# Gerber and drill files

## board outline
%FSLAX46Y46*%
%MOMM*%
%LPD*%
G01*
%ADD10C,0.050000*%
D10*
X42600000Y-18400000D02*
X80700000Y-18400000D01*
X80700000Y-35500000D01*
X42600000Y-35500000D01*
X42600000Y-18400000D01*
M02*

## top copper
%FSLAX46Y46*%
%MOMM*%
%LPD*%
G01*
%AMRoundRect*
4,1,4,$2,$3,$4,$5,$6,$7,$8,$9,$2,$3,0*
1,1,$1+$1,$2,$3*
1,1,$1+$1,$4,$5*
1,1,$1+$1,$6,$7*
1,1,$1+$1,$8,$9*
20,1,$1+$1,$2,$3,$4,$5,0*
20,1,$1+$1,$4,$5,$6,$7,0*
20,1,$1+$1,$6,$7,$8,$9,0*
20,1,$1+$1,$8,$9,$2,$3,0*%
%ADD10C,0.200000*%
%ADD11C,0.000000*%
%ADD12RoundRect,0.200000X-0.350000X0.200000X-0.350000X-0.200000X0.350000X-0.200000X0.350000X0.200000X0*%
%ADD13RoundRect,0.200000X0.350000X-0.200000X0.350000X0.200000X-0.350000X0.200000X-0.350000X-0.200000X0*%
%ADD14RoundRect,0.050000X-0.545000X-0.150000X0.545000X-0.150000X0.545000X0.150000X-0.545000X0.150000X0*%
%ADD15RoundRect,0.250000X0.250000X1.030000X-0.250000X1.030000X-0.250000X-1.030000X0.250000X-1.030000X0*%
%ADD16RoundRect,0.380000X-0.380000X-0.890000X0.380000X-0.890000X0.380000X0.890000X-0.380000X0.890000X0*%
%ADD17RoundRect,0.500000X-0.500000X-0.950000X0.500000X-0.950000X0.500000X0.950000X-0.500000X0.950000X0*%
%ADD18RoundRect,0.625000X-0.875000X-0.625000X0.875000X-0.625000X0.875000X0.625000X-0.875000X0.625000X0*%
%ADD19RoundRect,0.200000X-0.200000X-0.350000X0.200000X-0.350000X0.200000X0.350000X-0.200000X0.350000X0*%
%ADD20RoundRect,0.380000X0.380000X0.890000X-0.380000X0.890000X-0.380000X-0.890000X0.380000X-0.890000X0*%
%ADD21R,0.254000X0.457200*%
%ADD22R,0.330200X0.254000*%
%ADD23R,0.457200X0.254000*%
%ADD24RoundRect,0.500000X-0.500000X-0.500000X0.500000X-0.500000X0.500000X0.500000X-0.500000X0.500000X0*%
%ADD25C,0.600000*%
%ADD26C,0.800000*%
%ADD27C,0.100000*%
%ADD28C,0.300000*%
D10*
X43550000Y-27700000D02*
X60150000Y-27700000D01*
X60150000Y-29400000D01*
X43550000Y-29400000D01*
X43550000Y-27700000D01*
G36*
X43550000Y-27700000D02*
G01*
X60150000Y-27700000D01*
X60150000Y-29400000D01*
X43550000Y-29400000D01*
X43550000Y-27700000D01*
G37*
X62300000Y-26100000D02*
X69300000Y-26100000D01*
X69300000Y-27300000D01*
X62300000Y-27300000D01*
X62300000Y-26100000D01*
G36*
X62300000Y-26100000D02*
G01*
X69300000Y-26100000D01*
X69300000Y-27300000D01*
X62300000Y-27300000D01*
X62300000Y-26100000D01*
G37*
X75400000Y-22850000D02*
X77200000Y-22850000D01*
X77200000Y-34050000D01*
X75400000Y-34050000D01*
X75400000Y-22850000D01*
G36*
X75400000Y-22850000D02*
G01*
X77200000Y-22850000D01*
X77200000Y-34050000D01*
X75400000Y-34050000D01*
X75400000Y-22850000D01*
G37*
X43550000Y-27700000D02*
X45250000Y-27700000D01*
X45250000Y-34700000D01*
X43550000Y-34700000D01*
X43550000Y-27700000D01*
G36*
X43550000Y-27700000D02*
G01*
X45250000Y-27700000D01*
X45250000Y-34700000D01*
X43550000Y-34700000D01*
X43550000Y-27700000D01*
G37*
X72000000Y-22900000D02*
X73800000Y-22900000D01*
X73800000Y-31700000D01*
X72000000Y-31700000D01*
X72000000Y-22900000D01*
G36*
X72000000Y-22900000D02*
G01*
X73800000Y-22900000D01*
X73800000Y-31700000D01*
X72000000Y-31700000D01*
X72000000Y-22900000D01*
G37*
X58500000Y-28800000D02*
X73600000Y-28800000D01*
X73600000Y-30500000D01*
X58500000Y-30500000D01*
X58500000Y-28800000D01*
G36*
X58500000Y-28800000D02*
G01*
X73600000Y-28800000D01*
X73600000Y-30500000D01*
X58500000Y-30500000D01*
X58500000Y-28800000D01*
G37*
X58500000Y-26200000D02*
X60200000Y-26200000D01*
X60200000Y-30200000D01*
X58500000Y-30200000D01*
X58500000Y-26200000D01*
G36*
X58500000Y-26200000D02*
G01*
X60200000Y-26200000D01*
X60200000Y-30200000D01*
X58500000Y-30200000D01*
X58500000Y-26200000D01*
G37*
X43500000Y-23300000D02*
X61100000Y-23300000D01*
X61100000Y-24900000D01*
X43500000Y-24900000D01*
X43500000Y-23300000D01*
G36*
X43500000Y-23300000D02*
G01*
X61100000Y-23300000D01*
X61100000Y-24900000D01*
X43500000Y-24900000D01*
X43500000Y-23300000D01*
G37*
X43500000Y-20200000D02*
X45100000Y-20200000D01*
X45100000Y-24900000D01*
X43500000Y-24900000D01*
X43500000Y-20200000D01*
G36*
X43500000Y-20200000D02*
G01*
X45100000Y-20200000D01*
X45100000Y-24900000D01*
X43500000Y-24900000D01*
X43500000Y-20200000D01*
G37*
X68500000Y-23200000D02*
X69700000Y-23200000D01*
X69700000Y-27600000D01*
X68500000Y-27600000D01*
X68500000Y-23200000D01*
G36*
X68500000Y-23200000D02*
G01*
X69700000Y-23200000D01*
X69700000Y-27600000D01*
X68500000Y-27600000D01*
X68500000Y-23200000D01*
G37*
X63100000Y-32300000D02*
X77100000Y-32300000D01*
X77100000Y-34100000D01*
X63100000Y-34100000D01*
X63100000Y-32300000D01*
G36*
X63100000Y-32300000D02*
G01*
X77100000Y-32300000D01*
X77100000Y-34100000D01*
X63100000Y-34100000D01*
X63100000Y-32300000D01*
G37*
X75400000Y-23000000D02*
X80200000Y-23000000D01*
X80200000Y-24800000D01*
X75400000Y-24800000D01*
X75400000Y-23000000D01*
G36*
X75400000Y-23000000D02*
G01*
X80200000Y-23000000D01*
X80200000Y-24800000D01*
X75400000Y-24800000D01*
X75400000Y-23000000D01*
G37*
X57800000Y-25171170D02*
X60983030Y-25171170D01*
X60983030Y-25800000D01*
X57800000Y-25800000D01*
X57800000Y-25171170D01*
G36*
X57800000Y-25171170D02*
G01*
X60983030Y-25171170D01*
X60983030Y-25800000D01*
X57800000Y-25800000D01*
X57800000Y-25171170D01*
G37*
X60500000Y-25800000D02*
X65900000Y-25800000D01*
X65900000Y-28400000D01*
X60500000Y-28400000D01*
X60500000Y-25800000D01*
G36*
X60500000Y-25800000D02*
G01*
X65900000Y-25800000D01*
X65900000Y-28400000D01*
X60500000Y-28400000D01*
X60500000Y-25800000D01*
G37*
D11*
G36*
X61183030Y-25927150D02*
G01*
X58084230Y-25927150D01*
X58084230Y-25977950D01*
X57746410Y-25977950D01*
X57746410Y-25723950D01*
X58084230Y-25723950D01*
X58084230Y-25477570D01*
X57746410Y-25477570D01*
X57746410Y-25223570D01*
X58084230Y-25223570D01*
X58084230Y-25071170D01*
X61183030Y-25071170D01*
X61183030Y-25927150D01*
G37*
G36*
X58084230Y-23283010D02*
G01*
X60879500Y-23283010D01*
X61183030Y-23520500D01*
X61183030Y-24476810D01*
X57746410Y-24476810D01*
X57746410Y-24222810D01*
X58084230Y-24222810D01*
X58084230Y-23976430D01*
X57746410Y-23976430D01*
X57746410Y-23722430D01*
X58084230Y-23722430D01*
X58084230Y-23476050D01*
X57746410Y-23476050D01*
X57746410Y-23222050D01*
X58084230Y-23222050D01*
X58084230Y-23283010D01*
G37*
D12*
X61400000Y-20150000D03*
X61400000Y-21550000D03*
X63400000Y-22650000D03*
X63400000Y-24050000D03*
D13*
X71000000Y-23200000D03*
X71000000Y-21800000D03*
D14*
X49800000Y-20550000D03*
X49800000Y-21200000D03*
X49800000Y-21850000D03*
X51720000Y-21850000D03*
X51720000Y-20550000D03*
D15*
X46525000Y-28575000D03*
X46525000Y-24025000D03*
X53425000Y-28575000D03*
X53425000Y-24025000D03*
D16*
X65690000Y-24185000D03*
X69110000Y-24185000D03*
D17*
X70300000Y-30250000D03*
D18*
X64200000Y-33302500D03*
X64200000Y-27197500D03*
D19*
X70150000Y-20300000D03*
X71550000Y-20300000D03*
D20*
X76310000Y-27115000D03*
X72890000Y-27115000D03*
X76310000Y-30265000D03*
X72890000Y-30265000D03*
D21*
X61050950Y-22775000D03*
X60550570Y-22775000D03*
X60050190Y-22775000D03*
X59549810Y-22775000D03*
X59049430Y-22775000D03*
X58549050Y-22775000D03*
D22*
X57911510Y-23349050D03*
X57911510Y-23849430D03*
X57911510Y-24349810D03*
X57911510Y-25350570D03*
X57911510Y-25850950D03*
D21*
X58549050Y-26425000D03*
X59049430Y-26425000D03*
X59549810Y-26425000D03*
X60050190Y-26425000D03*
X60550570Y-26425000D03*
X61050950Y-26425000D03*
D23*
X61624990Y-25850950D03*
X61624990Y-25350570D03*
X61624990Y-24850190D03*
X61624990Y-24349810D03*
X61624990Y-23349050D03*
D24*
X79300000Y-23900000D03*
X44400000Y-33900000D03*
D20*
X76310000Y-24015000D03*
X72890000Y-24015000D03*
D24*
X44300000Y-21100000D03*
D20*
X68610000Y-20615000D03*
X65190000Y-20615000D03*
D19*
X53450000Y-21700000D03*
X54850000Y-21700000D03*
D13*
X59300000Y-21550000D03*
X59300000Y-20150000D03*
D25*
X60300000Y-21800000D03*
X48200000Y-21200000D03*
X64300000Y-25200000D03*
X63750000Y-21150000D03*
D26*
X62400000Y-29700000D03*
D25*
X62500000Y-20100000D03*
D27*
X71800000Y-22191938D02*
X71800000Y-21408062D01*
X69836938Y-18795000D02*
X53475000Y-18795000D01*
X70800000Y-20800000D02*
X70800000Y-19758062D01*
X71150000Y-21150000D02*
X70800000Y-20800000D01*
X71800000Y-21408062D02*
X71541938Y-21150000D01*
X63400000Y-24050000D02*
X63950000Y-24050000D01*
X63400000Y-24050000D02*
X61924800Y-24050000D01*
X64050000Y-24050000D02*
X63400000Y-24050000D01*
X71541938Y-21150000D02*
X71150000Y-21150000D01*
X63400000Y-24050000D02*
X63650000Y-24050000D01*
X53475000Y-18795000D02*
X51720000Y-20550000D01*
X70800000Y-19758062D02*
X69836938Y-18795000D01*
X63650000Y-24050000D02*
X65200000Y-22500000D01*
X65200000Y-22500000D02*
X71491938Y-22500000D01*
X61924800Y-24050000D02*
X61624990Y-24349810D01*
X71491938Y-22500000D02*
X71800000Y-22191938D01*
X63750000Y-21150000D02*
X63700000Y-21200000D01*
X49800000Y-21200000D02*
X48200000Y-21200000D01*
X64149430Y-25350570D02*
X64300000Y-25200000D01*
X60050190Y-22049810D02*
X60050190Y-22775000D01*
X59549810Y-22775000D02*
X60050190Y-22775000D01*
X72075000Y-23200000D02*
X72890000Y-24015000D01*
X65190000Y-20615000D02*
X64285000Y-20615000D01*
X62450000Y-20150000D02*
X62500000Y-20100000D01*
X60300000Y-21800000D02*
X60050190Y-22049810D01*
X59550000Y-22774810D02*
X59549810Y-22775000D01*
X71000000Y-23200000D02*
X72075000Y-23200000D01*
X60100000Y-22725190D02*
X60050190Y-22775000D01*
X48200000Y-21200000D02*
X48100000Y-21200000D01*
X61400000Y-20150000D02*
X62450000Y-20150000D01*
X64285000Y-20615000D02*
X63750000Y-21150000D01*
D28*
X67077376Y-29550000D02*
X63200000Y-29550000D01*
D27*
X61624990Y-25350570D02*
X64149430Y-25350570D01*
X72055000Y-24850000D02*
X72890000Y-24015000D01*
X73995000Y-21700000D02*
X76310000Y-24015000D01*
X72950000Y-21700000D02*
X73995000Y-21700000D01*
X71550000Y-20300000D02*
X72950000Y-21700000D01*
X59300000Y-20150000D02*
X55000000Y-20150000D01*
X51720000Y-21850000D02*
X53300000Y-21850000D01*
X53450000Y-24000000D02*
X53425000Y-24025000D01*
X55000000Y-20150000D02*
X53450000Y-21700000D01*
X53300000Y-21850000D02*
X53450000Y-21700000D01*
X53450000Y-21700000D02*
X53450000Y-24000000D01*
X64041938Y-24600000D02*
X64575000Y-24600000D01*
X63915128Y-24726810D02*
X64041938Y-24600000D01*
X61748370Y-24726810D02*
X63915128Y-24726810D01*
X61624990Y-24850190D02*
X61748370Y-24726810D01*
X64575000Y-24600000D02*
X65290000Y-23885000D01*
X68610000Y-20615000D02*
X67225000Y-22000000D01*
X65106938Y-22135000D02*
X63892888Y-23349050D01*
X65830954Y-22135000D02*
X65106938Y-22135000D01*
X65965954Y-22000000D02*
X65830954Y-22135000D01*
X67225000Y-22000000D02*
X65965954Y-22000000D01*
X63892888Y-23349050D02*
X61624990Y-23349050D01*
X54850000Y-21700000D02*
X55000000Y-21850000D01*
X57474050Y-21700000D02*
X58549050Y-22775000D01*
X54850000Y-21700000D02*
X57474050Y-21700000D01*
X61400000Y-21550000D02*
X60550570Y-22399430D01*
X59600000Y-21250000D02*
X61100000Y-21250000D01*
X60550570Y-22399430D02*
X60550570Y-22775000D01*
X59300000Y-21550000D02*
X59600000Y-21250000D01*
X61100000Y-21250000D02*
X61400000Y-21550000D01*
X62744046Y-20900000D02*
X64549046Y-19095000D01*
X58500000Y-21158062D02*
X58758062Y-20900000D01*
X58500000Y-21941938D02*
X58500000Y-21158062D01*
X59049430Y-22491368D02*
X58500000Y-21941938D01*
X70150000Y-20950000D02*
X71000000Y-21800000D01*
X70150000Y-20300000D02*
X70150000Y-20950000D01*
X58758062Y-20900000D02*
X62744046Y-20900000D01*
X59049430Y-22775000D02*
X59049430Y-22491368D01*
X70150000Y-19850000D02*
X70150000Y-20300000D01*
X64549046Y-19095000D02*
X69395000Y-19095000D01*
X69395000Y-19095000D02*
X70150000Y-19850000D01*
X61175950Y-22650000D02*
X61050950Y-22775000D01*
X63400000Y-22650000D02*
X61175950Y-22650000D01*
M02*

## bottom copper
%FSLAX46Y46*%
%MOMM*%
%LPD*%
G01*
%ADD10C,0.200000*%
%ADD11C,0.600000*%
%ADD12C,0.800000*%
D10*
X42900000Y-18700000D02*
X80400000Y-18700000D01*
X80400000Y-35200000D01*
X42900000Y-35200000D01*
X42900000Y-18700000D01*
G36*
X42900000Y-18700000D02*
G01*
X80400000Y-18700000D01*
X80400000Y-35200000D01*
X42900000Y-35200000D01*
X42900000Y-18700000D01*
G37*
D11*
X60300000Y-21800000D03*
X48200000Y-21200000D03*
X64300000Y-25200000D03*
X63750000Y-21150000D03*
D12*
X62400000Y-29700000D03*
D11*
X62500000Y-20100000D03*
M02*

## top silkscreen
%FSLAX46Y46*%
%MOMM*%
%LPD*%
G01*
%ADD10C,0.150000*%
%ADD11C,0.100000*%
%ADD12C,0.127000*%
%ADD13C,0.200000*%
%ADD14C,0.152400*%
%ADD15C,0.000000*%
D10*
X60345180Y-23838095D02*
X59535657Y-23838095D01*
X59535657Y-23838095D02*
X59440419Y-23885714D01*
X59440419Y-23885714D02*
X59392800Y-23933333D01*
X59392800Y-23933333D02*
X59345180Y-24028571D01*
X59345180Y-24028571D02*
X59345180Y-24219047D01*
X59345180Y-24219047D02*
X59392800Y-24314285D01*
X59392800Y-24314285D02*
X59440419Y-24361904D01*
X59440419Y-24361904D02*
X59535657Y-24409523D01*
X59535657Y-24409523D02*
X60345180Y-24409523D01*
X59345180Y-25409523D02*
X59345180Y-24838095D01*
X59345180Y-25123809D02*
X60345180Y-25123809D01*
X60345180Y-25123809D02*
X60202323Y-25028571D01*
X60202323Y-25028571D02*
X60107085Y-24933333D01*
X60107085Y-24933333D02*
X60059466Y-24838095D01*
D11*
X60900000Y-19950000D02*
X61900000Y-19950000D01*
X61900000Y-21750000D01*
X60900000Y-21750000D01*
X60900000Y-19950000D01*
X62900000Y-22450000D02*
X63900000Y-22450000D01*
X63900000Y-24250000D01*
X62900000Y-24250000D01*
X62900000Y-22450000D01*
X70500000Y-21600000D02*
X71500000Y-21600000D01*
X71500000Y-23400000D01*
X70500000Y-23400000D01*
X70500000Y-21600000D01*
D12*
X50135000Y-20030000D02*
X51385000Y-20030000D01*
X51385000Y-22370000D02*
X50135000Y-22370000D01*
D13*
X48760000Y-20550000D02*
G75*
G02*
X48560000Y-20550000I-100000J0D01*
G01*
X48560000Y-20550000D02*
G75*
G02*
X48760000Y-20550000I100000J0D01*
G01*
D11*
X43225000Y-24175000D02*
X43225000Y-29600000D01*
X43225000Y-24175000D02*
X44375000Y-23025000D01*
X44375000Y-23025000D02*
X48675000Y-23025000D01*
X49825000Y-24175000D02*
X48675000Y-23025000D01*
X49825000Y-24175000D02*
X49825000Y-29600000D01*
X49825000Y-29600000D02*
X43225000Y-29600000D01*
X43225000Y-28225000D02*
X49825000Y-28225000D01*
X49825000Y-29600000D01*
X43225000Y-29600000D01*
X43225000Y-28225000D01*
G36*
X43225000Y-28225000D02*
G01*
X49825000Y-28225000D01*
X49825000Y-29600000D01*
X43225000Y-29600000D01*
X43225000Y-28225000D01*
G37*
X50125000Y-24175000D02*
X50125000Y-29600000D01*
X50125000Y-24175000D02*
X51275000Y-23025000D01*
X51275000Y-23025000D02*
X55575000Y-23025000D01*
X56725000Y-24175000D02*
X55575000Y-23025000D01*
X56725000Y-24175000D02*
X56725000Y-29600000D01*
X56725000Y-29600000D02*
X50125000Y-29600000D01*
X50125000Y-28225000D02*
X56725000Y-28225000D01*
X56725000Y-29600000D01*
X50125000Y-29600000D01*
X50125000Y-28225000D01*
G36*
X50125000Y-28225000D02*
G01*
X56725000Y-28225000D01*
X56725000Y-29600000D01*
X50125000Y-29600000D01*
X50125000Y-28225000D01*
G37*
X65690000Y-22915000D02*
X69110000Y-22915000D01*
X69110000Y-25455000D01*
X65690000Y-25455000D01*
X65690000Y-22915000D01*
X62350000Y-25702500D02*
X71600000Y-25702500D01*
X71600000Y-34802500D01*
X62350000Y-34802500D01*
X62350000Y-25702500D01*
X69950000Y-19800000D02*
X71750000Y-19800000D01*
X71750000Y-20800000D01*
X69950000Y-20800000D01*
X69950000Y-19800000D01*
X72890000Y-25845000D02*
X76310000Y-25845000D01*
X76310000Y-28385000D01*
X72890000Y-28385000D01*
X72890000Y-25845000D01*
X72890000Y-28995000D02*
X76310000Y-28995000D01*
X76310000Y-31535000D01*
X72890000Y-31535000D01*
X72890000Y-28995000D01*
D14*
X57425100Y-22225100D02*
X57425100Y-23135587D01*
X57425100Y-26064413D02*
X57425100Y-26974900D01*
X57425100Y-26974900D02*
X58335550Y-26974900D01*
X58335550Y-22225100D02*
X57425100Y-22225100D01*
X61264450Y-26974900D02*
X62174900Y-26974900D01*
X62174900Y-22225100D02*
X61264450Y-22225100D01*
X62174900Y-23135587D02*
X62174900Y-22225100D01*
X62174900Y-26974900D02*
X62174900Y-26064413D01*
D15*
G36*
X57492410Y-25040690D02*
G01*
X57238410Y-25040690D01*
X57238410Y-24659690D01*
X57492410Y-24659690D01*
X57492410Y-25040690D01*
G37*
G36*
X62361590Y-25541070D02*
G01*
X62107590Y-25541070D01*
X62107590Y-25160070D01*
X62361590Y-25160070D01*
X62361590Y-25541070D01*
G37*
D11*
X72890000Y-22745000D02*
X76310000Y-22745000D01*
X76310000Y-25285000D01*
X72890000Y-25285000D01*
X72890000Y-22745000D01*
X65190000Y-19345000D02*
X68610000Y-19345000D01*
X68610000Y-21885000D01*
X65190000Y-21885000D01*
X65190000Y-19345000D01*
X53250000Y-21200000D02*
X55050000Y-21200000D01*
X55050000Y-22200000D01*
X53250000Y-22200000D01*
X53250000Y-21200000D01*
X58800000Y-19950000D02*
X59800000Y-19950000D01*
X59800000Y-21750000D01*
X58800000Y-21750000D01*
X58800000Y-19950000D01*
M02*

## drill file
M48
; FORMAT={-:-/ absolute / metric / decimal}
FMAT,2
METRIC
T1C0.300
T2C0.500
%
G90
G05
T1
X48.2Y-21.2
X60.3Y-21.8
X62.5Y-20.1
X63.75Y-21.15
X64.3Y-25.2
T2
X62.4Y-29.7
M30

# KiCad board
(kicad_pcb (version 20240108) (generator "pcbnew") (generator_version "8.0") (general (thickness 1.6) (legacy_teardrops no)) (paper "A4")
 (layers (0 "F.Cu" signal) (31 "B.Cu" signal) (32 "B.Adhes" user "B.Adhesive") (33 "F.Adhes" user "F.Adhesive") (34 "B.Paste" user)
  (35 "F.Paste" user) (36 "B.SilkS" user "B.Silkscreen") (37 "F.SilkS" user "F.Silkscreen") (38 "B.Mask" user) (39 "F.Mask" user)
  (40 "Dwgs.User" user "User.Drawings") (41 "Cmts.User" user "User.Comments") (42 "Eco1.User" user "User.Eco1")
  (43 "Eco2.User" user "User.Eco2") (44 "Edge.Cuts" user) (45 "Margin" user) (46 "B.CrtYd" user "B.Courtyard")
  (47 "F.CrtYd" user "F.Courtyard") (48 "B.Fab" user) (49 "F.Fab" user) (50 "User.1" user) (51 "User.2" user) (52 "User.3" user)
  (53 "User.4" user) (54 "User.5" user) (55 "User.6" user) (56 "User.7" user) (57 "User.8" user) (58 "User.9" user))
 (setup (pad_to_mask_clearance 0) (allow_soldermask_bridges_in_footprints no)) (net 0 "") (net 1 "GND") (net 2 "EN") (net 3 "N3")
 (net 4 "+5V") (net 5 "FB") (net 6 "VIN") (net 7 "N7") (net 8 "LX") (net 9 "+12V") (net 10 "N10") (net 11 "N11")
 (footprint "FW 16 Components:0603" (layer "F.Cu") (at 61.4 20.8 -90)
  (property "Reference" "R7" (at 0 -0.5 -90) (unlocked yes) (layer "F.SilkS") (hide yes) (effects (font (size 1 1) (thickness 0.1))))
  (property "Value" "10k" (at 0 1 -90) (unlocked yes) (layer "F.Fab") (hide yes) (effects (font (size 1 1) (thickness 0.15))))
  (fp_rect (start -0.85 -0.5) (end 0.95 0.5) (stroke (width 0.1) (type default)) (fill none) (layer "F.SilkS"))
  (pad "1" smd roundrect (at -0.65 0 270) (size 0.8 1.1) (layers "F.Cu" "F.Paste" "F.Mask") (roundrect_rratio 0.25) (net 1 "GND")
   (thermal_bridge_angle 45))
  (pad "2" smd roundrect (at 0.75 0 270) (size 0.8 1.1) (layers "F.Cu" "F.Paste" "F.Mask") (roundrect_rratio 0.25) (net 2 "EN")
   (thermal_bridge_angle 45)))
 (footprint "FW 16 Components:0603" (layer "F.Cu") (at 63.4 23.3 -90)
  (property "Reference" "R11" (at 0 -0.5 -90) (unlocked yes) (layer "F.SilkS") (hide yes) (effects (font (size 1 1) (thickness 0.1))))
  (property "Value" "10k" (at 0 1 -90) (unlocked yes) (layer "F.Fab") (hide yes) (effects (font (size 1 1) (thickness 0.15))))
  (fp_rect (start -0.85 -0.5) (end 0.95 0.5) (stroke (width 0.1) (type default)) (fill none) (layer "F.SilkS"))
  (pad "1" smd roundrect (at -0.65 0 270) (size 0.8 1.1) (layers "F.Cu" "F.Paste" "F.Mask") (roundrect_rratio 0.25) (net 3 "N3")
   (thermal_bridge_angle 45))
  (pad "2" smd roundrect (at 0.75 0 270) (size 0.8 1.1) (layers "F.Cu" "F.Paste" "F.Mask") (roundrect_rratio 0.25) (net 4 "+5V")
   (thermal_bridge_angle 45)))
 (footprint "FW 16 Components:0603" (layer "F.Cu") (at 71 22.55 90)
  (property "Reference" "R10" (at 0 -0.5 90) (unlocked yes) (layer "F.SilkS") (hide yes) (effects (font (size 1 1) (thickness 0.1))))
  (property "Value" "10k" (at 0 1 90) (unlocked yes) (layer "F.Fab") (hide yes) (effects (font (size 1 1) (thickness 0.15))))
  (fp_rect (start -0.85 -0.5) (end 0.95 0.5) (stroke (width 0.1) (type default)) (fill none) (layer "F.SilkS"))
  (pad "1" smd roundrect (at -0.65 0 90) (size 0.8 1.1) (layers "F.Cu" "F.Paste" "F.Mask") (roundrect_rratio 0.25) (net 1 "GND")
   (thermal_bridge_angle 45))
  (pad "2" smd roundrect (at 0.75 0 90) (size 0.8 1.1) (layers "F.Cu" "F.Paste" "F.Mask") (roundrect_rratio 0.25) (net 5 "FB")
   (thermal_bridge_angle 45)))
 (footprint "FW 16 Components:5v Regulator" (layer "F.Cu") (at 50.76 21.2)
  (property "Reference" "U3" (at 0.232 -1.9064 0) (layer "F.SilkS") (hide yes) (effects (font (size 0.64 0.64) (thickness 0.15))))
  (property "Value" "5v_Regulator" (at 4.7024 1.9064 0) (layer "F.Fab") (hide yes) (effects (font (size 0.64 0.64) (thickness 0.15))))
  (fp_line (start -0.625 -1.17) (end 0.625 -1.17) (stroke (width 0.127) (type solid)) (layer "F.SilkS"))
  (fp_line (start 0.625 1.17) (end -0.625 1.17) (stroke (width 0.127) (type solid)) (layer "F.SilkS"))
  (fp_circle (center -2.1 -0.65) (end -2 -0.65) (stroke (width 0.2) (type solid)) (fill none) (layer "F.SilkS"))
  (pad "1" smd roundrect (at -0.96 -0.65) (size 1.19 0.4) (layers "F.Cu" "F.Paste" "F.Mask") (roundrect_rratio 0.125)
   (solder_mask_margin 0.102))
  (pad "2" smd roundrect (at -0.96 0) (size 1.19 0.4) (layers "F.Cu" "F.Paste" "F.Mask") (roundrect_rratio 0.125) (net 1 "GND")
   (solder_mask_margin 0.102))
  (pad "3" smd roundrect (at -0.96 0.65) (size 1.19 0.4) (layers "F.Cu" "F.Paste" "F.Mask") (roundrect_rratio 0.125)
   (solder_mask_margin 0.102))
  (pad "4" smd roundrect (at 0.96 0.65) (size 1.19 0.4) (layers "F.Cu" "F.Paste" "F.Mask") (roundrect_rratio 0.125) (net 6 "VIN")
   (solder_mask_margin 0.102))
  (pad "5" smd roundrect (at 0.96 -0.65) (size 1.19 0.4) (layers "F.Cu" "F.Paste" "F.Mask") (roundrect_rratio 0.125) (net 4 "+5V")
   (solder_mask_margin 0.102)))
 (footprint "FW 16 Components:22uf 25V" (layer "F.Cu") (at 49.975 26.125 90)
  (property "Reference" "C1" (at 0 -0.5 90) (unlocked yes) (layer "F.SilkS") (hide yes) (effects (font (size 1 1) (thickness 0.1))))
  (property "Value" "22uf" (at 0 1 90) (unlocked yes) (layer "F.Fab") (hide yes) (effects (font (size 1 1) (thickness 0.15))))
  (fp_line (start 1.95 -6.75) (end -3.475 -6.75) (stroke (width 0.1) (type default)) (layer "F.SilkS"))
  (fp_line (start 1.95 -6.75) (end 3.1 -5.6) (stroke (width 0.1) (type default)) (layer "F.SilkS"))
  (fp_line (start 3.1 -5.6) (end 3.1 -1.3) (stroke (width 0.1) (type default)) (layer "F.SilkS"))
  (fp_line (start 1.95 -0.15) (end 3.1 -1.3) (stroke (width 0.1) (type default)) (layer "F.SilkS"))
  (fp_line (start 1.95 -0.15) (end -3.475 -0.15) (stroke (width 0.1) (type default)) (layer "F.SilkS"))
  (fp_line (start -3.475 -0.15) (end -3.475 -6.75) (stroke (width 0.1) (type default)) (layer "F.SilkS"))
  (fp_rect (start -3.475 -6.75) (end -2.1 -0.15) (stroke (width 0.1) (type solid)) (fill solid) (layer "F.SilkS"))
  (pad "1" smd roundrect (at -2.45 -3.45 180) (size 1 2.56) (layers "F.Cu" "F.Paste" "F.Mask") (roundrect_rratio 0.25) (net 1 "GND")
   (thermal_bridge_angle 45))
  (pad "2" smd roundrect (at 2.1 -3.45 180) (size 1 2.56) (layers "F.Cu" "F.Paste" "F.Mask") (roundrect_rratio 0.25) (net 6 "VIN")
   (thermal_bridge_angle 45)))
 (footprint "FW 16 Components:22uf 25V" (layer "F.Cu") (at 56.875 26.125 90)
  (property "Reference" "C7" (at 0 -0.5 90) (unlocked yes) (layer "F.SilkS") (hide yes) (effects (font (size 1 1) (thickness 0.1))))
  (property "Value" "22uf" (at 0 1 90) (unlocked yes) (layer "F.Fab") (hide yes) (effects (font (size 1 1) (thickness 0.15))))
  (fp_line (start 1.95 -6.75) (end -3.475 -6.75) (stroke (width 0.1) (type default)) (layer "F.SilkS"))
  (fp_line (start 1.95 -6.75) (end 3.1 -5.6) (stroke (width 0.1) (type default)) (layer "F.SilkS"))
  (fp_line (start 3.1 -5.6) (end 3.1 -1.3) (stroke (width 0.1) (type default)) (layer "F.SilkS"))
  (fp_line (start 1.95 -0.15) (end 3.1 -1.3) (stroke (width 0.1) (type default)) (layer "F.SilkS"))
  (fp_line (start 1.95 -0.15) (end -3.475 -0.15) (stroke (width 0.1) (type default)) (layer "F.SilkS"))
  (fp_line (start -3.475 -0.15) (end -3.475 -6.75) (stroke (width 0.1) (type default)) (layer "F.SilkS"))
  (fp_rect (start -3.475 -6.75) (end -2.1 -0.15) (stroke (width 0.1) (type solid)) (fill solid) (layer "F.SilkS"))
  (pad "1" smd roundrect (at -2.45 -3.45 180) (size 1 2.56) (layers "F.Cu" "F.Paste" "F.Mask") (roundrect_rratio 0.25) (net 1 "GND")
   (thermal_bridge_angle 45))
  (pad "2" smd roundrect (at 2.1 -3.45 180) (size 1 2.56) (layers "F.Cu" "F.Paste" "F.Mask") (roundrect_rratio 0.25) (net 6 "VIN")
   (thermal_bridge_angle 45)))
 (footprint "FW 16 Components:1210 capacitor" (layer "F.Cu") (at 67.56 26.685)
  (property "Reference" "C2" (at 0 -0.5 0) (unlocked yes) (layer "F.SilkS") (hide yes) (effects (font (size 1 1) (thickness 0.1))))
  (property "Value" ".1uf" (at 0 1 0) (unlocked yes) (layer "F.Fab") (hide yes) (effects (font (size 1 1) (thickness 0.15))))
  (fp_rect (start -1.87 -3.77) (end 1.55 -1.23) (stroke (width 0.1) (type default)) (fill none) (layer "F.SilkS"))
  (pad "1" smd roundrect (at -1.87 -2.5) (size 1.52 2.54) (layers "F.Cu" "F.Paste" "F.Mask") (roundrect_rratio 0.25) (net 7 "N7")
   (thermal_bridge_angle 45))
  (pad "2" smd roundrect (at 1.55 -2.5) (size 1.52 2.54) (layers "F.Cu" "F.Paste" "F.Mask") (roundrect_rratio 0.25) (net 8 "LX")
   (thermal_bridge_angle 45)))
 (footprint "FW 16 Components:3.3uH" (layer "F.Cu") (at 66.8 30.2)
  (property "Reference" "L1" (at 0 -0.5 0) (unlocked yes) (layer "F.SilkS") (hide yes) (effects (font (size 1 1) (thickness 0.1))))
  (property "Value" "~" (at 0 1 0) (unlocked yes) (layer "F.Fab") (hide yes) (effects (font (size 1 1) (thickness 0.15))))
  (fp_rect (start -4.45 -4.4975) (end 4.8 4.6025) (stroke (width 0.1) (type default)) (fill none) (layer "F.SilkS"))
  (pad "" smd roundrect (at 3.5 0.05) (size 2 2.9) (layers "F.Cu" "F.Paste" "F.Mask") (roundrect_rratio 0.25) (thermal_bridge_angle 45))
  (pad "1" smd roundrect (at -2.6 3.1025) (size 3 2.5) (layers "F.Cu" "F.Paste" "F.Mask") (roundrect_rratio 0.25) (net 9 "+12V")
   (thermal_bridge_angle 45))
  (pad "2" smd roundrect (at -2.6 -3.0025) (size 3 2.5) (layers "F.Cu" "F.Paste" "F.Mask") (roundrect_rratio 0.25) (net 8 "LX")
   (thermal_bridge_angle 45)))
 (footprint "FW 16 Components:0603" (layer "F.Cu") (at 70.8 20.3)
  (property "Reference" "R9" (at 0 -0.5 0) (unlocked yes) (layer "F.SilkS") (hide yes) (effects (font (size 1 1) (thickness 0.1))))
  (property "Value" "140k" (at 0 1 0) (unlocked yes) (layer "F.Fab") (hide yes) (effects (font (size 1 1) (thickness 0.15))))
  (fp_rect (start -0.85 -0.5) (end 0.95 0.5) (stroke (width 0.1) (type default)) (fill none) (layer "F.SilkS"))
  (pad "1" smd roundrect (at -0.65 0) (size 0.8 1.1) (layers "F.Cu" "F.Paste" "F.Mask") (roundrect_rratio 0.25) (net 5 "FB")
   (thermal_bridge_angle 45))
  (pad "2" smd roundrect (at 0.75 0) (size 0.8 1.1) (layers "F.Cu" "F.Paste" "F.Mask") (roundrect_rratio 0.25) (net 9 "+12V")
   (thermal_bridge_angle 45)))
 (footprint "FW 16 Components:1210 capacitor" (layer "F.Cu") (at 74.44 24.615 180)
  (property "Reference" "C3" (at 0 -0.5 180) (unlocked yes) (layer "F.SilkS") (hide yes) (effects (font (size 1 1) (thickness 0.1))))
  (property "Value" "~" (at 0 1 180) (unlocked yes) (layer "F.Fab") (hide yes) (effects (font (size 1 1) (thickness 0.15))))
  (fp_rect (start -1.87 -3.77) (end 1.55 -1.23) (stroke (width 0.1) (type default)) (fill none) (layer "F.SilkS"))
  (pad "1" smd roundrect (at -1.87 -2.5 180) (size 1.52 2.54) (layers "F.Cu" "F.Paste" "F.Mask") (roundrect_rratio 0.25) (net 9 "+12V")
   (thermal_bridge_angle 45))
  (pad "2" smd roundrect (at 1.55 -2.5 180) (size 1.52 2.54) (layers "F.Cu" "F.Paste" "F.Mask") (roundrect_rratio 0.25) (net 1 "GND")
   (thermal_bridge_angle 45)))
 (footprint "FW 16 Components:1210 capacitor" (layer "F.Cu") (at 74.44 27.765 180)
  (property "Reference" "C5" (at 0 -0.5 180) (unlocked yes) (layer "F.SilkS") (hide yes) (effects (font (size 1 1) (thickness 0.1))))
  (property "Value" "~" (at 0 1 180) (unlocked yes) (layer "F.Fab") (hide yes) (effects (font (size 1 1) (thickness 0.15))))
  (fp_rect (start -1.87 -3.77) (end 1.55 -1.23) (stroke (width 0.1) (type default)) (fill none) (layer "F.SilkS"))
  (pad "1" smd roundrect (at -1.87 -2.5 180) (size 1.52 2.54) (layers "F.Cu" "F.Paste" "F.Mask") (roundrect_rratio 0.25) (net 9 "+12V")
   (thermal_bridge_angle 45))
  (pad "2" smd roundrect (at 1.55 -2.5 180) (size 1.52 2.54) (layers "F.Cu" "F.Paste" "F.Mask") (roundrect_rratio 0.25) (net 1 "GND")
   (thermal_bridge_angle 45)))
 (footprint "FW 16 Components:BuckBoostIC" (layer "F.Cu") (at 59.8 24.6 -90)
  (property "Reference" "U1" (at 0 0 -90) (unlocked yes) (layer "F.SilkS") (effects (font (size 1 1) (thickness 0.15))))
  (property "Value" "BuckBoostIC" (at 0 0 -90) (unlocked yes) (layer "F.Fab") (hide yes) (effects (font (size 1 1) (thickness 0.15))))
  (fp_poly
   (pts (xy 0.47117 1.71577) (xy 0.62357 1.71577) (xy 0.62357 2.05359) (xy 0.87757 2.05359) (xy 0.87757 1.71577) (xy 1.12395 1.71577)
    (xy 1.12395 2.05359) (xy 1.37795 2.05359) (xy 1.37795 1.71577) (xy 1.32715 1.71577) (xy 1.32715 -1.38303) (xy 0.47117 -1.38303))
   (stroke (width 0) (type solid)) (fill solid) (layer "F.Cu"))
  (fp_poly
   (pts (xy -1.37795 2.05359) (xy -1.37795 1.71577) (xy -1.31699 1.71577) (xy -1.31699 -1.0795) (xy -1.0795 -1.38303) (xy -0.12319 -1.38303)
    (xy -0.12319 2.05359) (xy -0.37719 2.05359) (xy -0.37719 1.71577) (xy -0.62357 1.71577) (xy -0.62357 2.05359) (xy -0.87757 2.05359)
    (xy -0.87757 1.71577) (xy -1.12395 1.71577) (xy -1.12395 2.05359))
   (stroke (width 0) (type solid)) (fill solid) (layer "F.Cu"))
  (fp_line (start -2.3749 2.3749) (end -1.464413 2.3749) (stroke (width 0.1524) (type solid)) (layer "F.SilkS"))
  (fp_line (start 1.464413 2.3749) (end 2.3749 2.3749) (stroke (width 0.1524) (type solid)) (layer "F.SilkS"))
  (fp_line (start 2.3749 2.3749) (end 2.3749 1.46445) (stroke (width 0.1524) (type solid)) (layer "F.SilkS"))
  (fp_line (start -2.3749 1.46445) (end -2.3749 2.3749) (stroke (width 0.1524) (type solid)) (layer "F.SilkS"))
  (fp_line (start 2.3749 -1.46445) (end 2.3749 -2.3749) (stroke (width 0.1524) (type solid)) (layer "F.SilkS"))
  (fp_line (start -2.3749 -2.3749) (end -2.3749 -1.46445) (stroke (width 0.1524) (type solid)) (layer "F.SilkS"))
  (fp_line (start -1.464413 -2.3749) (end -2.3749 -2.3749) (stroke (width 0.1524) (type solid)) (layer "F.SilkS"))
  (fp_line (start 2.3749 -2.3749) (end 1.464413 -2.3749) (stroke (width 0.1524) (type solid)) (layer "F.SilkS"))
  (fp_poly
   (pts (xy 0.05969 2.30759) (xy 0.05969 2.56159) (xy 0.44069 2.56159) (xy 0.44069 2.30759)) (stroke (width 0) (type solid)) (fill solid)
   (layer "F.SilkS"))
  (fp_poly
   (pts (xy 0.56007 -2.30759) (xy 0.56007 -2.56159) (xy 0.94107 -2.56159) (xy 0.94107 -2.30759)) (stroke (width 0) (type solid))
   (fill solid) (layer "F.SilkS"))
  (pad "1" smd rect (at -1.825 -1.25095) (size 0.254 0.4572) (layers "F.Cu" "F.Paste" "F.Mask") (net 3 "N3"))
  (pad "2" smd rect (at -1.825 -0.75057) (size 0.254 0.4572) (layers "F.Cu" "F.Paste" "F.Mask") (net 2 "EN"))
  (pad "3" smd rect (at -1.825 -0.25019) (size 0.254 0.4572) (layers "F.Cu" "F.Paste" "F.Mask") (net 1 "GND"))
  (pad "4" smd rect (at -1.825 0.25019) (size 0.254 0.4572) (layers "F.Cu" "F.Paste" "F.Mask") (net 1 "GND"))
  (pad "5" smd rect (at -1.825 0.75057) (size 0.254 0.4572) (layers "F.Cu" "F.Paste" "F.Mask") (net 5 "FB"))
  (pad "6" smd rect (at -1.825 1.25095) (size 0.254 0.4572) (layers "F.Cu" "F.Paste" "F.Mask") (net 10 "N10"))
  (pad "7" smd rect (at -1.25095 1.88849 270) (size 0.254 0.3302) (layers "F.Cu" "F.Paste" "F.Mask") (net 6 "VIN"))
  (pad "8" smd rect (at -0.75057 1.88849 270) (size 0.254 0.3302) (layers "F.Cu" "F.Paste" "F.Mask") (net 6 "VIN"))
  (pad "9" smd rect (at -0.25019 1.88849 270) (size 0.254 0.3302) (layers "F.Cu" "F.Paste" "F.Mask") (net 6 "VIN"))
  (pad "10" smd rect (at 0.75057 1.88849 270) (size 0.254 0.3302) (layers "F.Cu" "F.Paste" "F.Mask") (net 8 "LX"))
  (pad "11" smd rect (at 1.25095 1.88849 270) (size 0.254 0.3302) (layers "F.Cu" "F.Paste" "F.Mask") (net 8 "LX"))
  (pad "12" smd rect (at 1.825 1.25095) (size 0.254 0.4572) (layers "F.Cu" "F.Paste" "F.Mask") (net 1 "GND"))
  (pad "13" smd rect (at 1.825 0.75057) (size 0.254 0.4572) (layers "F.Cu" "F.Paste" "F.Mask") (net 1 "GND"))
  (pad "14" smd rect (at 1.825 0.25019) (size 0.254 0.4572) (layers "F.Cu" "F.Paste" "F.Mask") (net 1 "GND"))
  (pad "15" smd rect (at 1.825 -0.25019) (size 0.254 0.4572) (layers "F.Cu" "F.Paste" "F.Mask") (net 1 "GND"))
  (pad "16" smd rect (at 1.825 -0.75057) (size 0.254 0.4572) (layers "F.Cu" "F.Paste" "F.Mask") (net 8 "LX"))
  (pad "17" smd rect (at 1.825 -1.25095) (size 0.254 0.4572) (layers "F.Cu" "F.Paste" "F.Mask") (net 8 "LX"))
  (pad "18" smd rect (at 1.25095 -1.82499 270) (size 0.254 0.4572) (layers "F.Cu" "F.Paste" "F.Mask") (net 8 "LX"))
  (pad "19" smd rect (at 0.75057 -1.82499 270) (size 0.254 0.4572) (layers "F.Cu" "F.Paste" "F.Mask") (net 1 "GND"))
  (pad "20" smd rect (at 0.25019 -1.82499 270) (size 0.254 0.4572) (layers "F.Cu" "F.Paste" "F.Mask") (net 7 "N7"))
  (pad "21" smd rect (at -0.25019 -1.82499 270) (size 0.254 0.4572) (layers "F.Cu" "F.Paste" "F.Mask") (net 4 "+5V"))
  (pad "22" smd rect (at -1.25095 -1.82499 270) (size 0.254 0.4572) (layers "F.Cu" "F.Paste" "F.Mask") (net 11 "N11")))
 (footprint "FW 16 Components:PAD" (layer "F.Cu") (at 79.35 26.45)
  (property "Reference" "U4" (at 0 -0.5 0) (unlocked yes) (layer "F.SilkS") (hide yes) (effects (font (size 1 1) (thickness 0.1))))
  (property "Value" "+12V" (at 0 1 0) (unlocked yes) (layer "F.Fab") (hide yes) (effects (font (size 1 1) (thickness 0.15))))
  (pad "1" smd roundrect (at -0.05 -2.55) (size 2 2) (layers "F.Cu" "F.Paste" "F.Mask") (roundrect_rratio 0.25) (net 9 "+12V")
   (thermal_bridge_angle 45)))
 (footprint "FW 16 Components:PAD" (layer "F.Cu") (at 44.45 36.45)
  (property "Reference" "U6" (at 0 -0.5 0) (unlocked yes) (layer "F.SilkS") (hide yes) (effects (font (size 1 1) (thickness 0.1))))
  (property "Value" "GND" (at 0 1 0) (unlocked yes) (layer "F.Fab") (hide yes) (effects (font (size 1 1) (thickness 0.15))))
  (pad "1" smd roundrect (at -0.05 -2.55) (size 2 2) (layers "F.Cu" "F.Paste" "F.Mask") (roundrect_rratio 0.25) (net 1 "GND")
   (thermal_bridge_angle 45)))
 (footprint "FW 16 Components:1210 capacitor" (layer "F.Cu") (at 74.44 21.515 180)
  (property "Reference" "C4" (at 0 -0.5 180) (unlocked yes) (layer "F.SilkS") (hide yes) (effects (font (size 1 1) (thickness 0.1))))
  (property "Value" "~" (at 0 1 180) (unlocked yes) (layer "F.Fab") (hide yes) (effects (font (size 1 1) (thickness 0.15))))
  (fp_rect (start -1.87 -3.77) (end 1.55 -1.23) (stroke (width 0.1) (type default)) (fill none) (layer "F.SilkS"))
  (pad "1" smd roundrect (at -1.87 -2.5 180) (size 1.52 2.54) (layers "F.Cu" "F.Paste" "F.Mask") (roundrect_rratio 0.25) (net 9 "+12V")
   (thermal_bridge_angle 45))
  (pad "2" smd roundrect (at 1.55 -2.5 180) (size 1.52 2.54) (layers "F.Cu" "F.Paste" "F.Mask") (roundrect_rratio 0.25) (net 1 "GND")
   (thermal_bridge_angle 45)))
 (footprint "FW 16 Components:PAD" (layer "F.Cu") (at 44.35 23.65)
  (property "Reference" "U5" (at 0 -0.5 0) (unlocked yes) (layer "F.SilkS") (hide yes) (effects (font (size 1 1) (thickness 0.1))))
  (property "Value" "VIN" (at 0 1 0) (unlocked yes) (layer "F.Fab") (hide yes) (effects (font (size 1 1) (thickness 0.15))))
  (pad "1" smd roundrect (at -0.05 -2.55) (size 2 2) (layers "F.Cu" "F.Paste" "F.Mask") (roundrect_rratio 0.25) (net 6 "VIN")
   (thermal_bridge_angle 45)))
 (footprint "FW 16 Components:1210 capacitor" (layer "F.Cu") (at 66.74 18.115 180)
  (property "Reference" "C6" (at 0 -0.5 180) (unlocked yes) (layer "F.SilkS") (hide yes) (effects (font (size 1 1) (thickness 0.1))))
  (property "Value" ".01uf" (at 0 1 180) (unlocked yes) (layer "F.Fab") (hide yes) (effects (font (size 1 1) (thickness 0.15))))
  (fp_rect (start -1.87 -3.77) (end 1.55 -1.23) (stroke (width 0.1) (type default)) (fill none) (layer "F.SilkS"))
  (pad "1" smd roundrect (at -1.87 -2.5 180) (size 1.52 2.54) (layers "F.Cu" "F.Paste" "F.Mask") (roundrect_rratio 0.25) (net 11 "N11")
   (thermal_bridge_angle 45))
  (pad "2" smd roundrect (at 1.55 -2.5 180) (size 1.52 2.54) (layers "F.Cu" "F.Paste" "F.Mask") (roundrect_rratio 0.25) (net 1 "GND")
   (thermal_bridge_angle 45)))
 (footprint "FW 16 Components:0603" (layer "F.Cu") (at 54.1 21.7)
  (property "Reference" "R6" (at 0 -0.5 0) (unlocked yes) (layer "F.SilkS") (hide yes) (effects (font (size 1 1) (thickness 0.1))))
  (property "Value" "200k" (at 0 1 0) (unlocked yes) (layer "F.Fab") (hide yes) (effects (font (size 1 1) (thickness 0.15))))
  (fp_rect (start -0.85 -0.5) (end 0.95 0.5) (stroke (width 0.1) (type default)) (fill none) (layer "F.SilkS"))
  (pad "1" smd roundrect (at -0.65 0) (size 0.8 1.1) (layers "F.Cu" "F.Paste" "F.Mask") (roundrect_rratio 0.25) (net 6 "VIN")
   (thermal_bridge_angle 45))
  (pad "2" smd roundrect (at 0.75 0) (size 0.8 1.1) (layers "F.Cu" "F.Paste" "F.Mask") (roundrect_rratio 0.25) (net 10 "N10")
   (thermal_bridge_angle 45)))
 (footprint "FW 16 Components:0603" (layer "F.Cu") (at 59.3 20.9 90)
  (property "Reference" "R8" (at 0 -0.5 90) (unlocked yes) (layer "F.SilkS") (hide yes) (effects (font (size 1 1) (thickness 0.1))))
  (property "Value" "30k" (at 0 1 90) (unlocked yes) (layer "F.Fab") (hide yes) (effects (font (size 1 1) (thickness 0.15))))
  (fp_rect (start -0.85 -0.5) (end 0.95 0.5) (stroke (width 0.1) (type default)) (fill none) (layer "F.SilkS"))
  (pad "1" smd roundrect (at -0.65 0 90) (size 0.8 1.1) (layers "F.Cu" "F.Paste" "F.Mask") (roundrect_rratio 0.25) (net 2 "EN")
   (thermal_bridge_angle 45))
  (pad "2" smd roundrect (at 0.75 0 90) (size 0.8 1.1) (layers "F.Cu" "F.Paste" "F.Mask") (roundrect_rratio 0.25) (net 6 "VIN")
   (thermal_bridge_angle 45)))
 (gr_rect (start 43.55 27.7) (end 60.15 29.4) (stroke (width 0.2) (type solid)) (fill solid) (layer "F.Cu") (net 1))
 (gr_rect (start 62.3 26.1) (end 69.3 27.3) (stroke (width 0.2) (type solid)) (fill solid) (layer "F.Cu") (net 8))
 (gr_rect (start 75.4 22.85) (end 77.2 34.05) (stroke (width 0.2) (type solid)) (fill solid) (layer "F.Cu") (net 9))
 (gr_rect (start 43.55 27.7) (end 45.25 34.7) (stroke (width 0.2) (type solid)) (fill solid) (layer "F.Cu") (net 1))
 (gr_rect (start 72 22.9) (end 73.8 31.7) (stroke (width 0.2) (type solid)) (fill solid) (layer "F.Cu") (net 1))
 (gr_rect (start 58.5 28.8) (end 73.6 30.5) (stroke (width 0.2) (type solid)) (fill solid) (layer "F.Cu") (net 1))
 (gr_rect (start 58.5 26.2) (end 60.2 30.2) (stroke (width 0.2) (type solid)) (fill solid) (layer "F.Cu") (net 1))
 (gr_rect (start 43.5 23.3) (end 61.1 24.9) (stroke (width 0.2) (type solid)) (fill solid) (layer "F.Cu") (net 6))
 (gr_rect (start 43.5 20.2) (end 45.1 24.9) (stroke (width 0.2) (type solid)) (fill solid) (layer "F.Cu") (net 6))
 (gr_rect (start 68.5 23.2) (end 69.7 27.6) (stroke (width 0.2) (type solid)) (fill solid) (layer "F.Cu") (net 8))
 (gr_rect (start 63.1 32.3) (end 77.1 34.1) (stroke (width 0.2) (type solid)) (fill solid) (layer "F.Cu") (net 9))
 (gr_rect (start 75.4 23) (end 80.2 24.8) (stroke (width 0.2) (type solid)) (fill solid) (layer "F.Cu") (net 9))
 (gr_rect (start 57.8 25.17117) (end 60.98303 25.8) (stroke (width 0.2) (type solid)) (fill solid) (layer "F.Cu") (net 8))
 (gr_rect (start 60.5 25.8) (end 65.9 28.4) (stroke (width 0.2) (type solid)) (fill solid) (layer "F.Cu") (net 8))
 (gr_rect (start 42.9 18.7) (end 80.4 35.2) (stroke (width 0.2) (type solid)) (fill solid) (layer "B.Cu") (net 1))
 (gr_rect (start 42.6 18.4) (end 80.7 35.5) (stroke (width 0.05) (type default)) (fill none) (layer "Edge.Cuts"))
 (segment (start 71.8 22.191938) (end 71.8 21.408062) (width 0.1) (layer "F.Cu") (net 4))
 (segment (start 69.836938 18.795) (end 53.475 18.795) (width 0.1) (layer "F.Cu") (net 4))
 (segment (start 70.8 20.8) (end 70.8 19.758062) (width 0.1) (layer "F.Cu") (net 4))
 (segment (start 71.15 21.15) (end 70.8 20.8) (width 0.1) (layer "F.Cu") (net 4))
 (segment (start 71.8 21.408062) (end 71.541938 21.15) (width 0.1) (layer "F.Cu") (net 4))
 (segment (start 63.4 24.05) (end 63.95 24.05) (width 0.1) (layer "F.Cu") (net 4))
 (segment (start 63.4 24.05) (end 61.9248 24.05) (width 0.1) (layer "F.Cu") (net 4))
 (segment (start 64.05 24.05) (end 63.4 24.05) (width 0.1) (layer "F.Cu") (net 4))
 (segment (start 71.541938 21.15) (end 71.15 21.15) (width 0.1) (layer "F.Cu") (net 4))
 (segment (start 63.4 24.05) (end 63.65 24.05) (width 0.1) (layer "F.Cu") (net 4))
 (segment (start 53.475 18.795) (end 51.72 20.55) (width 0.1) (layer "F.Cu") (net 4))
 (segment (start 70.8 19.758062) (end 69.836938 18.795) (width 0.1) (layer "F.Cu") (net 4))
 (segment (start 63.65 24.05) (end 65.2 22.5) (width 0.1) (layer "F.Cu") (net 4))
 (segment (start 65.2 22.5) (end 71.491938 22.5) (width 0.1) (layer "F.Cu") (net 4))
 (segment (start 61.9248 24.05) (end 61.62499 24.34981) (width 0.1) (layer "F.Cu") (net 4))
 (segment (start 71.491938 22.5) (end 71.8 22.191938) (width 0.1) (layer "F.Cu") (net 4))
 (segment (start 63.75 21.15) (end 63.7 21.2) (width 0.1) (layer "F.Cu") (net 1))
 (segment (start 49.8 21.2) (end 48.2 21.2) (width 0.1) (layer "F.Cu") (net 1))
 (segment (start 64.14943 25.35057) (end 64.3 25.2) (width 0.1) (layer "F.Cu") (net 1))
 (segment (start 60.05019 22.04981) (end 60.05019 22.775) (width 0.1) (layer "F.Cu") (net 1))
 (segment (start 59.54981 22.775) (end 60.05019 22.775) (width 0.1) (layer "F.Cu") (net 1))
 (segment (start 72.075 23.2) (end 72.89 24.015) (width 0.1) (layer "F.Cu") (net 1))
 (segment (start 65.19 20.615) (end 64.285 20.615) (width 0.1) (layer "F.Cu") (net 1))
 (segment (start 62.45 20.15) (end 62.5 20.1) (width 0.1) (layer "F.Cu") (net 1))
 (segment (start 60.3 21.8) (end 60.05019 22.04981) (width 0.1) (layer "F.Cu") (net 1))
 (segment (start 59.55 22.77481) (end 59.54981 22.775) (width 0.1) (layer "F.Cu") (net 1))
 (segment (start 71 23.2) (end 72.075 23.2) (width 0.1) (layer "F.Cu") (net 1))
 (segment (start 60.1 22.72519) (end 60.05019 22.775) (width 0.1) (layer "F.Cu") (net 1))
 (segment (start 48.2 21.2) (end 48.1 21.2) (width 0.1) (layer "F.Cu") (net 1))
 (segment (start 61.4 20.15) (end 62.45 20.15) (width 0.1) (layer "F.Cu") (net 1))
 (segment (start 64.285 20.615) (end 63.75 21.15) (width 0.1) (layer "F.Cu") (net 1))
 (segment (start 67.077376 29.55) (end 63.2 29.55) (width 0.3) (layer "F.Cu") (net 1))
 (segment (start 61.62499 25.35057) (end 64.14943 25.35057) (width 0.1) (layer "F.Cu") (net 1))
 (segment (start 72.055 24.85) (end 72.89 24.015) (width 0.1) (layer "F.Cu") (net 1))
 (via (at 60.3 21.8) (size 0.6) (drill 0.3) (layers "F.Cu" "B.Cu") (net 1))
 (via (at 48.2 21.2) (size 0.6) (drill 0.3) (layers "F.Cu" "B.Cu") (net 1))
 (via (at 64.3 25.2) (size 0.6) (drill 0.3) (layers "F.Cu" "B.Cu") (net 1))
 (via (at 63.75 21.15) (size 0.6) (drill 0.3) (layers "F.Cu" "B.Cu") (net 1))
 (via (at 62.4 29.7) (size 0.8) (drill 0.5) (layers "F.Cu" "B.Cu") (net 1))
 (via (at 62.5 20.1) (size 0.6) (drill 0.3) (layers "F.Cu" "B.Cu") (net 1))
 (segment (start 73.995 21.7) (end 76.31 24.015) (width 0.1) (layer "F.Cu") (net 9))
 (segment (start 72.95 21.7) (end 73.995 21.7) (width 0.1) (layer "F.Cu") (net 9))
 (segment (start 71.55 20.3) (end 72.95 21.7) (width 0.1) (layer "F.Cu") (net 9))
 (segment (start 59.3 20.15) (end 55 20.15) (width 0.1) (layer "F.Cu") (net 6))
 (segment (start 51.72 21.85) (end 53.3 21.85) (width 0.1) (layer "F.Cu") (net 6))
 (segment (start 53.45 24) (end 53.425 24.025) (width 0.1) (layer "F.Cu") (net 6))
 (segment (start 55 20.15) (end 53.45 21.7) (width 0.1) (layer "F.Cu") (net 6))
 (segment (start 53.3 21.85) (end 53.45 21.7) (width 0.1) (layer "F.Cu") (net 6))
 (segment (start 53.45 21.7) (end 53.45 24) (width 0.1) (layer "F.Cu") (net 6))
 (segment (start 64.041938 24.6) (end 64.575 24.6) (width 0.1) (layer "F.Cu") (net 7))
 (segment (start 63.915128 24.72681) (end 64.041938 24.6) (width 0.1) (layer "F.Cu") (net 7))
 (segment (start 61.74837 24.72681) (end 63.915128 24.72681) (width 0.1) (layer "F.Cu") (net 7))
 (segment (start 61.62499 24.85019) (end 61.74837 24.72681) (width 0.1) (layer "F.Cu") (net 7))
 (segment (start 64.575 24.6) (end 65.29 23.885) (width 0.1) (layer "F.Cu") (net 7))
 (segment (start 68.61 20.615) (end 67.225 22) (width 0.1) (layer "F.Cu") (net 11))
 (segment (start 65.106938 22.135) (end 63.892888 23.34905) (width 0.1) (layer "F.Cu") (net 11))
 (segment (start 65.830954 22.135) (end 65.106938 22.135) (width 0.1) (layer "F.Cu") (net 11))
 (segment (start 65.965954 22) (end 65.830954 22.135) (width 0.1) (layer "F.Cu") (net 11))
 (segment (start 67.225 22) (end 65.965954 22) (width 0.1) (layer "F.Cu") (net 11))
 (segment (start 63.892888 23.34905) (end 61.62499 23.34905) (width 0.1) (layer "F.Cu") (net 11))
 (segment (start 54.85 21.7) (end 55 21.85) (width 0.1) (layer "F.Cu") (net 10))
 (segment (start 57.47405 21.7) (end 58.54905 22.775) (width 0.1) (layer "F.Cu") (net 10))
 (segment (start 54.85 21.7) (end 57.47405 21.7) (width 0.1) (layer "F.Cu") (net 10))
 (segment (start 61.4 21.55) (end 60.55057 22.39943) (width 0.1) (layer "F.Cu") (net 2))
 (segment (start 59.6 21.25) (end 61.1 21.25) (width 0.1) (layer "F.Cu") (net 2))
 (segment (start 60.55057 22.39943) (end 60.55057 22.775) (width 0.1) (layer "F.Cu") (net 2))
 (segment (start 59.3 21.55) (end 59.6 21.25) (width 0.1) (layer "F.Cu") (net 2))
 (segment (start 61.1 21.25) (end 61.4 21.55) (width 0.1) (layer "F.Cu") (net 2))
 (segment (start 62.744046 20.9) (end 64.549046 19.095) (width 0.1) (layer "F.Cu") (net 5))
 (segment (start 58.5 21.158062) (end 58.758062 20.9) (width 0.1) (layer "F.Cu") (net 5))
 (segment (start 58.5 21.941938) (end 58.5 21.158062) (width 0.1) (layer "F.Cu") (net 5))
 (segment (start 59.04943 22.491368) (end 58.5 21.941938) (width 0.1) (layer "F.Cu") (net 5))
 (segment (start 70.15 20.95) (end 71 21.8) (width 0.1) (layer "F.Cu") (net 5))
 (segment (start 70.15 20.3) (end 70.15 20.95) (width 0.1) (layer "F.Cu") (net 5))
 (segment (start 58.758062 20.9) (end 62.744046 20.9) (width 0.1) (layer "F.Cu") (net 5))
 (segment (start 59.04943 22.775) (end 59.04943 22.491368) (width 0.1) (layer "F.Cu") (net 5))
 (segment (start 70.15 19.85) (end 70.15 20.3) (width 0.1) (layer "F.Cu") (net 5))
 (segment (start 64.549046 19.095) (end 69.395 19.095) (width 0.1) (layer "F.Cu") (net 5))
 (segment (start 69.395 19.095) (end 70.15 19.85) (width 0.1) (layer "F.Cu") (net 5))
 (segment (start 61.17595 22.65) (end 61.05095 22.775) (width 0.1) (layer "F.Cu") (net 3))
 (segment (start 63.4 22.65) (end 61.17595 22.65) (width 0.1) (layer "F.Cu") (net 3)))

